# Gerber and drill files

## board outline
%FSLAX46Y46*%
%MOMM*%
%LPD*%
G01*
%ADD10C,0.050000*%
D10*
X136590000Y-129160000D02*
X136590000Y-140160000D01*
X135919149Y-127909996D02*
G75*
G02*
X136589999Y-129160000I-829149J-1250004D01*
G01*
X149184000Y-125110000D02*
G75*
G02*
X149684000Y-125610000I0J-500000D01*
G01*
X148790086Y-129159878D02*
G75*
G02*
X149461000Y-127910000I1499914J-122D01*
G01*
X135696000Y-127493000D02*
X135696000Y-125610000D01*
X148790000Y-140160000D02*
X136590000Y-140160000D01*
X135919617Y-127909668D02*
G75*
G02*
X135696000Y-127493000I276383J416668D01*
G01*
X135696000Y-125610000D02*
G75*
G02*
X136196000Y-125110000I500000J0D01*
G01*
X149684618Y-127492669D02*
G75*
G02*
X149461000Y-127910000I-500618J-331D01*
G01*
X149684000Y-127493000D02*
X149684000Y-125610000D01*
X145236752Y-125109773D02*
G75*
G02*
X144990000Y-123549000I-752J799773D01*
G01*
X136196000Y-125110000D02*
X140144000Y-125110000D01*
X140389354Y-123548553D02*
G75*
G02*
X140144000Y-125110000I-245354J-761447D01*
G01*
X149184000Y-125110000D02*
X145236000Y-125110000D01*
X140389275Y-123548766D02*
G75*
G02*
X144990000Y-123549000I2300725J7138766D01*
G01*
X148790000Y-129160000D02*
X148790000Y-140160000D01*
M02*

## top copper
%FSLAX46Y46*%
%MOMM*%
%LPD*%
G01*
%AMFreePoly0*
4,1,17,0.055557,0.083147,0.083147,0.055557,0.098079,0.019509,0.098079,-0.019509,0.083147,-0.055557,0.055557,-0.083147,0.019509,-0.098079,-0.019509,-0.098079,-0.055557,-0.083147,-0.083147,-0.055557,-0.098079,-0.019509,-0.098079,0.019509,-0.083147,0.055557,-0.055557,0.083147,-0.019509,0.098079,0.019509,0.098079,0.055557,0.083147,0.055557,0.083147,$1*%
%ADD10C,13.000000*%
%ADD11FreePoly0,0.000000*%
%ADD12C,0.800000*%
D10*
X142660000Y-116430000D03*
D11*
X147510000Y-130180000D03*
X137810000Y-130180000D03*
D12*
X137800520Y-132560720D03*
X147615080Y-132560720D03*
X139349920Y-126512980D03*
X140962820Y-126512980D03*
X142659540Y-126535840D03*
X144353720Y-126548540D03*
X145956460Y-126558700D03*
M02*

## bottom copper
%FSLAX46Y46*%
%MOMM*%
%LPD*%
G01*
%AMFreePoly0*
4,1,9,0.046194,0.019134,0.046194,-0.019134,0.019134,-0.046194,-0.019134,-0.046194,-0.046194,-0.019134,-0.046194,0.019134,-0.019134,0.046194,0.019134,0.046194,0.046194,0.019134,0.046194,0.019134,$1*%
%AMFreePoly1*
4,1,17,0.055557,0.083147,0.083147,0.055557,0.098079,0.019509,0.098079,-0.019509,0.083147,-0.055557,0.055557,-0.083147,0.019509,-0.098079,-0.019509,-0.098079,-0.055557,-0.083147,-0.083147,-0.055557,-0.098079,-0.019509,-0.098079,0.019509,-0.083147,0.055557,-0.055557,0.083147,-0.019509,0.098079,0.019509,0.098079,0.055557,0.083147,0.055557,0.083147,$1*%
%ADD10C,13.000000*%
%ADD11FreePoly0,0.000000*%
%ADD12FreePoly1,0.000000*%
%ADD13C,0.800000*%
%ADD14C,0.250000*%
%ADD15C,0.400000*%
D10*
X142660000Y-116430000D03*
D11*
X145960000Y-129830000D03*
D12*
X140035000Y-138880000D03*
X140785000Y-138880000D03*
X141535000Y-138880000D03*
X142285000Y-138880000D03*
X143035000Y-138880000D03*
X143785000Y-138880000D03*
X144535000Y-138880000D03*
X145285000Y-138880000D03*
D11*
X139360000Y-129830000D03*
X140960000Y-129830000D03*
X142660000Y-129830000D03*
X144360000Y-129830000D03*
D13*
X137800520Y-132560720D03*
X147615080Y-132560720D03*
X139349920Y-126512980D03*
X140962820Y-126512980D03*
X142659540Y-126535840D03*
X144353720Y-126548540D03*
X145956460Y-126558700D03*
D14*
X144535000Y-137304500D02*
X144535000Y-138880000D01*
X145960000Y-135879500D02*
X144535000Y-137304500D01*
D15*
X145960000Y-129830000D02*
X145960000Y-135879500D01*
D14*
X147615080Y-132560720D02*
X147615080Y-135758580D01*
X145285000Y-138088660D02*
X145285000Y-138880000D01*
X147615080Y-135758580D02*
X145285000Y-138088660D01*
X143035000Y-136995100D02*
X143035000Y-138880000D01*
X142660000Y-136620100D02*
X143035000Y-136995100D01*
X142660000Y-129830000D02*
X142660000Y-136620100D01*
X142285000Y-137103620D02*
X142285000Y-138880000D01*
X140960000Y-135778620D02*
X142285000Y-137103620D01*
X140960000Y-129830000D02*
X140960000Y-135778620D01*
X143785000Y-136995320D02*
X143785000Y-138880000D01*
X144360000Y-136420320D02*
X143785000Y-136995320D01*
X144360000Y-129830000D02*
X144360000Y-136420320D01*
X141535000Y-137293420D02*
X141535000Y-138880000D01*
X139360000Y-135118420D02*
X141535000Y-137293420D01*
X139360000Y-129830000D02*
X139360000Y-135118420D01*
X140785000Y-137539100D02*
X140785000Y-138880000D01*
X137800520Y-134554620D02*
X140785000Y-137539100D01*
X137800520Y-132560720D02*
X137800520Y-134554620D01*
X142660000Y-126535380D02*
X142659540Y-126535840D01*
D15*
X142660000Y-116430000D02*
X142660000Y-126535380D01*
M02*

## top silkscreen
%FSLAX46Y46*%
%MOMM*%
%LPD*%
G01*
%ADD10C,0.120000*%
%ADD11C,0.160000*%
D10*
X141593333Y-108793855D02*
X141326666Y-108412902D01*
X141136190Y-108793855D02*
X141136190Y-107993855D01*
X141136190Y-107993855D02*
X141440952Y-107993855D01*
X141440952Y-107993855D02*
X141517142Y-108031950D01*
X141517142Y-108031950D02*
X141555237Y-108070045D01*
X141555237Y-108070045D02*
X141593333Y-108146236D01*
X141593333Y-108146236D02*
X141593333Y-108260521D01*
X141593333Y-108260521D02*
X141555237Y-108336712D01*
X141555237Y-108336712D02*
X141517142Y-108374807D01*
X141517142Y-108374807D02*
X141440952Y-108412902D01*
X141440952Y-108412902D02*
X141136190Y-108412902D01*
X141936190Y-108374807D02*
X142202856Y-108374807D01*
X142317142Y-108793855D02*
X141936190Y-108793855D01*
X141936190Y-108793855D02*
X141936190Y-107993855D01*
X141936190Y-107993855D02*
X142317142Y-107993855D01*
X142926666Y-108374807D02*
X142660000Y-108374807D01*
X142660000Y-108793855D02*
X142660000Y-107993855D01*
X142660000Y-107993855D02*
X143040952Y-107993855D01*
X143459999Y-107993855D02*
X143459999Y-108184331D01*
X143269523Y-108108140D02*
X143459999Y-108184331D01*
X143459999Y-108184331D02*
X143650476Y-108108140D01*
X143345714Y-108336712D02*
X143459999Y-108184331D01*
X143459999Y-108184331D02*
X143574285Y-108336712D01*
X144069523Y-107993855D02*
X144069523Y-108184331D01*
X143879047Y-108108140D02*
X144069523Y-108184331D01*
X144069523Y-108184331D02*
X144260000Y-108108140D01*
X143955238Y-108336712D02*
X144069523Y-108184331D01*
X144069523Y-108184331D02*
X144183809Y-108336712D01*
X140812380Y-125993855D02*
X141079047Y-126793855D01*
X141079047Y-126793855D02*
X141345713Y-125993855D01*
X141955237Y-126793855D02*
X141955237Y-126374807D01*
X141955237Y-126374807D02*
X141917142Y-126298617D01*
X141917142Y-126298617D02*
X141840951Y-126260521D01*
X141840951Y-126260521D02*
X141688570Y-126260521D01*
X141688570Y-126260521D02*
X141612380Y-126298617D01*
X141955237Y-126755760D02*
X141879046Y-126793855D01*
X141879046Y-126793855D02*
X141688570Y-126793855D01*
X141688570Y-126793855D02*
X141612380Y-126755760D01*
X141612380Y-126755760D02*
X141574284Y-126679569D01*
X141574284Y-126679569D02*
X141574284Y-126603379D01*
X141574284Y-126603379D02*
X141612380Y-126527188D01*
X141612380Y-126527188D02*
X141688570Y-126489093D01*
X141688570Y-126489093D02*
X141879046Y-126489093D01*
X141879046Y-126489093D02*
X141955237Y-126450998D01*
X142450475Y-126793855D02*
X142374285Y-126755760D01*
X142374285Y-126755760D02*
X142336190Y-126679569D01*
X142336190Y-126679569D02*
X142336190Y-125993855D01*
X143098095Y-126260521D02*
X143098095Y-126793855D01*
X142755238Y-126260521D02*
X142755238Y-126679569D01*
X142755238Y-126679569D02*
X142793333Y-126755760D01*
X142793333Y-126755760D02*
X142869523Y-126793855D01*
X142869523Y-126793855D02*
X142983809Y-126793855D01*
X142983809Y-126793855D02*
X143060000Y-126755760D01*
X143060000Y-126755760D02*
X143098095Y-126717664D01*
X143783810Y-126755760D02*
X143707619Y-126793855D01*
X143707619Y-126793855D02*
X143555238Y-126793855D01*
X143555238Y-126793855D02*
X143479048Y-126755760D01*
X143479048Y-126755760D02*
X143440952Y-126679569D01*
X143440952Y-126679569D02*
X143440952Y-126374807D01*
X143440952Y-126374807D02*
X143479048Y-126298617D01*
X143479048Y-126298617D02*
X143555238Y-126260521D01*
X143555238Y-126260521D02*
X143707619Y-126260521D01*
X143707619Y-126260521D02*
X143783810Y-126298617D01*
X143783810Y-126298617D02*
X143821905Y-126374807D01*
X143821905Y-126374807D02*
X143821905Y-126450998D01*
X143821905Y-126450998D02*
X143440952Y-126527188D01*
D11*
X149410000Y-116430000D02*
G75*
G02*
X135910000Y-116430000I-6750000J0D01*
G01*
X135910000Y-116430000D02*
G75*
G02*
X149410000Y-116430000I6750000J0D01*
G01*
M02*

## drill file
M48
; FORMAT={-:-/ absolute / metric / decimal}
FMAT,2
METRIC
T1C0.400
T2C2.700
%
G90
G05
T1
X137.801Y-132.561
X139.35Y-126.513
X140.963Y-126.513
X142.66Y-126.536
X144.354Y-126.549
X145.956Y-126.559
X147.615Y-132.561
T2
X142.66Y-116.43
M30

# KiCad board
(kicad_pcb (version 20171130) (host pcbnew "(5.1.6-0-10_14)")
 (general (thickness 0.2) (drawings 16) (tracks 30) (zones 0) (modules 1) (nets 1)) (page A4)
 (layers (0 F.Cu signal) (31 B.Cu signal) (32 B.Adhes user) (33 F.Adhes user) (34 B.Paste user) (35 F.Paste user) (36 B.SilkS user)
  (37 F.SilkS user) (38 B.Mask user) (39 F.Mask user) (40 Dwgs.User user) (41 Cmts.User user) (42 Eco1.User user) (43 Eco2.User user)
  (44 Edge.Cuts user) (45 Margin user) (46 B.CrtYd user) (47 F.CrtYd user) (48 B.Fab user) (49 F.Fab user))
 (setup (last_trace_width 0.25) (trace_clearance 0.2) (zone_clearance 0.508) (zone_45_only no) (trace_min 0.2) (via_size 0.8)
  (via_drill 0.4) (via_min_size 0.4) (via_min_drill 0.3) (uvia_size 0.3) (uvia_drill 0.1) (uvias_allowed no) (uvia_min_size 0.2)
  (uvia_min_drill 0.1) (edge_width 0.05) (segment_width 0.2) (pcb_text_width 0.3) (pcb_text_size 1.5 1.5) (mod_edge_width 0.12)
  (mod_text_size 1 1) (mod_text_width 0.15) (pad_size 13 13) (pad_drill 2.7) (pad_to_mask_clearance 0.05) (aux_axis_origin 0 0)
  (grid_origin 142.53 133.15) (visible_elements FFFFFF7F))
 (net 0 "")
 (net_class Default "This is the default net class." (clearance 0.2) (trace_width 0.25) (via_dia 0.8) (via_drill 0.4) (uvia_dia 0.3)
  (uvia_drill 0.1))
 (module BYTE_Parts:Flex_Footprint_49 (layer F.Cu) (at 142.66 116.43)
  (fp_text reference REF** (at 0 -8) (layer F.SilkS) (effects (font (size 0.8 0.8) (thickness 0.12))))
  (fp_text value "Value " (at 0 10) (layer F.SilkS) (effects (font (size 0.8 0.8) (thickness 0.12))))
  (fp_circle (center 0 0) (end -6.75 0) (layer F.SilkS) (width 0.16))
  (pad "#" thru_hole circle (at 0 0) (size 13 13) (drill 2.7) (layers *.Cu *.Mask))
  (pad "#" smd custom (at 3.3 13.4) (size 0.1 0.1) (layers B.Cu B.Mask) (zone_connect 0) (options (clearance outline) (anchor circle))
   (primitives))
  (pad "#" smd custom (at -2.625 22.45) (size 0.2 0.2) (layers B.Cu B.Mask) (zone_connect 0) (options (clearance outline) (anchor circle))
   (primitives))
  (pad "#" smd custom (at -1.875 22.45) (size 0.2 0.2) (layers B.Cu B.Mask) (zone_connect 0) (options (clearance outline) (anchor circle))
   (primitives))
  (pad "#" smd custom (at -1.125 22.45) (size 0.2 0.2) (layers B.Cu B.Mask) (zone_connect 0) (options (clearance outline) (anchor circle))
   (primitives))
  (pad "#" smd custom (at -0.375 22.45) (size 0.2 0.2) (layers B.Cu B.Mask) (zone_connect 0) (options (clearance outline) (anchor circle))
   (primitives))
  (pad "#" smd custom (at 0.375 22.45) (size 0.2 0.2) (layers B.Cu B.Mask) (zone_connect 0) (options (clearance outline) (anchor circle))
   (primitives))
  (pad "#" smd custom (at 1.125 22.45) (size 0.2 0.2) (layers B.Cu B.Mask) (zone_connect 0) (options (clearance outline) (anchor circle))
   (primitives))
  (pad "#" smd custom (at 1.875 22.45) (size 0.2 0.2) (layers B.Cu B.Mask) (zone_connect 0) (options (clearance outline) (anchor circle))
   (primitives))
  (pad "#" smd custom (at 2.625 22.45) (size 0.2 0.2) (layers B.Cu B.Mask) (zone_connect 0) (options (clearance outline) (anchor circle))
   (primitives))
  (pad "#" smd custom (at 4.85 13.75) (size 0.2 0.2) (layers F.Cu F.Mask) (zone_connect 0) (options (clearance outline) (anchor circle))
   (primitives))
  (pad "#" smd custom (at -4.85 13.75) (size 0.2 0.2) (layers F.Cu F.Mask) (zone_connect 0) (options (clearance outline) (anchor circle))
   (primitives))
  (pad "#" smd custom (at -3.3 13.4) (size 0.1 0.1) (layers B.Cu B.Mask) (zone_connect 0) (options (clearance outline) (anchor circle))
   (primitives))
  (pad "#" smd custom (at -1.7 13.4) (size 0.1 0.1) (layers B.Cu B.Mask) (zone_connect 0) (options (clearance outline) (anchor circle))
   (primitives))
  (pad "#" smd custom (at 0 13.4) (size 0.1 0.1) (layers B.Cu B.Mask) (zone_connect 0) (options (clearance outline) (anchor circle))
   (primitives))
  (pad "#" smd custom (at 1.7 13.4) (size 0.1 0.1) (layers B.Cu B.Mask) (zone_connect 0) (options (clearance outline) (anchor circle))
   (primitives)))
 (gr_line (start 136.59 129.16) (end 136.59 140.16) (angle 90) (layer Edge.Cuts) (width 0.05))
 (gr_arc (start 135.09 129.16) (end 136.59 129.16) (angle -56.443) (layer Edge.Cuts) (width 0.05))
 (gr_arc (start 149.184 125.61) (end 149.684 125.61) (angle -90) (layer Edge.Cuts) (width 0.05))
 (gr_arc (start 150.29 129.16) (end 149.461 127.91) (angle -56.443) (layer Edge.Cuts) (width 0.05))
 (gr_line (start 135.696 127.493) (end 135.696 125.61) (angle 90) (layer Edge.Cuts) (width 0.05))
 (gr_line (start 148.79 140.16) (end 136.59 140.16) (angle 90) (layer Edge.Cuts) (width 0.05))
 (gr_arc (start 136.196 127.493) (end 135.696 127.493) (angle -56.443) (layer Edge.Cuts) (width 0.05))
 (gr_arc (start 136.196 125.61) (end 136.196 125.11) (angle -90) (layer Edge.Cuts) (width 0.05))
 (gr_arc (start 149.184 127.493) (end 149.461 127.91) (angle -56.443) (layer Edge.Cuts) (width 0.05))
 (gr_line (start 149.684 127.493) (end 149.684 125.61) (angle 90) (layer Edge.Cuts) (width 0.05))
 (gr_arc (start 145.236 124.31) (end 144.99 123.549) (angle -162.14) (layer Edge.Cuts) (width 0.05))
 (gr_line (start 136.196 125.11) (end 140.144 125.11) (angle 90) (layer Edge.Cuts) (width 0.05))
 (gr_arc (start 140.144 124.31) (end 140.144 125.11) (angle -162.14) (layer Edge.Cuts) (width 0.05))
 (gr_line (start 149.184 125.11) (end 145.236 125.11) (angle 90) (layer Edge.Cuts) (width 0.05))
 (gr_arc (start 142.69 116.41) (end 144.99 123.549) (angle -324.279) (layer Edge.Cuts) (width 0.05))
 (gr_line (start 148.79 129.16) (end 148.79 140.16) (angle 90) (layer Edge.Cuts) (width 0.05))
 (segment (start 144.535 137.3045) (end 144.535 138.88) (width 0.25) (layer B.Cu) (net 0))
 (segment (start 145.96 135.8795) (end 144.535 137.3045) (width 0.25) (layer B.Cu) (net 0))
 (segment (start 145.96 129.83) (end 145.96 135.8795) (width 0.4) (layer B.Cu) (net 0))
 (via (at 137.80052 132.56072) (size 0.8) (drill 0.4) (layers F.Cu B.Cu) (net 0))
 (via (at 147.61508 132.56072) (size 0.8) (drill 0.4) (layers F.Cu B.Cu) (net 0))
 (segment (start 147.61508 132.56072) (end 147.61508 135.75858) (width 0.25) (layer B.Cu) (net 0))
 (segment (start 145.285 138.08866) (end 145.285 138.88) (width 0.25) (layer B.Cu) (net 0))
 (segment (start 147.61508 135.75858) (end 145.285 138.08866) (width 0.25) (layer B.Cu) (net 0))
 (segment (start 143.035 136.9951) (end 143.035 138.88) (width 0.25) (layer B.Cu) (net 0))
 (segment (start 142.66 136.6201) (end 143.035 136.9951) (width 0.25) (layer B.Cu) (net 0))
 (segment (start 142.66 129.83) (end 142.66 136.6201) (width 0.25) (layer B.Cu) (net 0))
 (segment (start 142.285 137.10362) (end 142.285 138.88) (width 0.25) (layer B.Cu) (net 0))
 (segment (start 140.96 135.77862) (end 142.285 137.10362) (width 0.25) (layer B.Cu) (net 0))
 (segment (start 140.96 129.83) (end 140.96 135.77862) (width 0.25) (layer B.Cu) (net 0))
 (segment (start 143.785 136.99532) (end 143.785 138.88) (width 0.25) (layer B.Cu) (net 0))
 (segment (start 144.36 136.42032) (end 143.785 136.99532) (width 0.25) (layer B.Cu) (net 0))
 (segment (start 144.36 129.83) (end 144.36 136.42032) (width 0.25) (layer B.Cu) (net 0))
 (segment (start 141.535 137.29342) (end 141.535 138.88) (width 0.25) (layer B.Cu) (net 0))
 (segment (start 139.36 135.11842) (end 141.535 137.29342) (width 0.25) (layer B.Cu) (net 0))
 (segment (start 139.36 129.83) (end 139.36 135.11842) (width 0.25) (layer B.Cu) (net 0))
 (segment (start 140.785 137.5391) (end 140.785 138.88) (width 0.25) (layer B.Cu) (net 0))
 (segment (start 137.80052 134.55462) (end 140.785 137.5391) (width 0.25) (layer B.Cu) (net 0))
 (segment (start 137.80052 132.56072) (end 137.80052 134.55462) (width 0.25) (layer B.Cu) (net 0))
 (via (at 139.34992 126.51298) (size 0.8) (drill 0.4) (layers F.Cu B.Cu) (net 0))
 (via (at 140.96282 126.51298) (size 0.8) (drill 0.4) (layers F.Cu B.Cu) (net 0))
 (via (at 142.65954 126.53584) (size 0.8) (drill 0.4) (layers F.Cu B.Cu) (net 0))
 (via (at 144.35372 126.54854) (size 0.8) (drill 0.4) (layers F.Cu B.Cu) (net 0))
 (via (at 145.95646 126.5587) (size 0.8) (drill 0.4) (layers F.Cu B.Cu) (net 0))
 (segment (start 142.66 126.53538) (end 142.65954 126.53584) (width 0.25) (layer B.Cu) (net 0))
 (segment (start 142.66 116.43) (end 142.66 126.53538) (width 0.4) (layer B.Cu) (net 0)))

